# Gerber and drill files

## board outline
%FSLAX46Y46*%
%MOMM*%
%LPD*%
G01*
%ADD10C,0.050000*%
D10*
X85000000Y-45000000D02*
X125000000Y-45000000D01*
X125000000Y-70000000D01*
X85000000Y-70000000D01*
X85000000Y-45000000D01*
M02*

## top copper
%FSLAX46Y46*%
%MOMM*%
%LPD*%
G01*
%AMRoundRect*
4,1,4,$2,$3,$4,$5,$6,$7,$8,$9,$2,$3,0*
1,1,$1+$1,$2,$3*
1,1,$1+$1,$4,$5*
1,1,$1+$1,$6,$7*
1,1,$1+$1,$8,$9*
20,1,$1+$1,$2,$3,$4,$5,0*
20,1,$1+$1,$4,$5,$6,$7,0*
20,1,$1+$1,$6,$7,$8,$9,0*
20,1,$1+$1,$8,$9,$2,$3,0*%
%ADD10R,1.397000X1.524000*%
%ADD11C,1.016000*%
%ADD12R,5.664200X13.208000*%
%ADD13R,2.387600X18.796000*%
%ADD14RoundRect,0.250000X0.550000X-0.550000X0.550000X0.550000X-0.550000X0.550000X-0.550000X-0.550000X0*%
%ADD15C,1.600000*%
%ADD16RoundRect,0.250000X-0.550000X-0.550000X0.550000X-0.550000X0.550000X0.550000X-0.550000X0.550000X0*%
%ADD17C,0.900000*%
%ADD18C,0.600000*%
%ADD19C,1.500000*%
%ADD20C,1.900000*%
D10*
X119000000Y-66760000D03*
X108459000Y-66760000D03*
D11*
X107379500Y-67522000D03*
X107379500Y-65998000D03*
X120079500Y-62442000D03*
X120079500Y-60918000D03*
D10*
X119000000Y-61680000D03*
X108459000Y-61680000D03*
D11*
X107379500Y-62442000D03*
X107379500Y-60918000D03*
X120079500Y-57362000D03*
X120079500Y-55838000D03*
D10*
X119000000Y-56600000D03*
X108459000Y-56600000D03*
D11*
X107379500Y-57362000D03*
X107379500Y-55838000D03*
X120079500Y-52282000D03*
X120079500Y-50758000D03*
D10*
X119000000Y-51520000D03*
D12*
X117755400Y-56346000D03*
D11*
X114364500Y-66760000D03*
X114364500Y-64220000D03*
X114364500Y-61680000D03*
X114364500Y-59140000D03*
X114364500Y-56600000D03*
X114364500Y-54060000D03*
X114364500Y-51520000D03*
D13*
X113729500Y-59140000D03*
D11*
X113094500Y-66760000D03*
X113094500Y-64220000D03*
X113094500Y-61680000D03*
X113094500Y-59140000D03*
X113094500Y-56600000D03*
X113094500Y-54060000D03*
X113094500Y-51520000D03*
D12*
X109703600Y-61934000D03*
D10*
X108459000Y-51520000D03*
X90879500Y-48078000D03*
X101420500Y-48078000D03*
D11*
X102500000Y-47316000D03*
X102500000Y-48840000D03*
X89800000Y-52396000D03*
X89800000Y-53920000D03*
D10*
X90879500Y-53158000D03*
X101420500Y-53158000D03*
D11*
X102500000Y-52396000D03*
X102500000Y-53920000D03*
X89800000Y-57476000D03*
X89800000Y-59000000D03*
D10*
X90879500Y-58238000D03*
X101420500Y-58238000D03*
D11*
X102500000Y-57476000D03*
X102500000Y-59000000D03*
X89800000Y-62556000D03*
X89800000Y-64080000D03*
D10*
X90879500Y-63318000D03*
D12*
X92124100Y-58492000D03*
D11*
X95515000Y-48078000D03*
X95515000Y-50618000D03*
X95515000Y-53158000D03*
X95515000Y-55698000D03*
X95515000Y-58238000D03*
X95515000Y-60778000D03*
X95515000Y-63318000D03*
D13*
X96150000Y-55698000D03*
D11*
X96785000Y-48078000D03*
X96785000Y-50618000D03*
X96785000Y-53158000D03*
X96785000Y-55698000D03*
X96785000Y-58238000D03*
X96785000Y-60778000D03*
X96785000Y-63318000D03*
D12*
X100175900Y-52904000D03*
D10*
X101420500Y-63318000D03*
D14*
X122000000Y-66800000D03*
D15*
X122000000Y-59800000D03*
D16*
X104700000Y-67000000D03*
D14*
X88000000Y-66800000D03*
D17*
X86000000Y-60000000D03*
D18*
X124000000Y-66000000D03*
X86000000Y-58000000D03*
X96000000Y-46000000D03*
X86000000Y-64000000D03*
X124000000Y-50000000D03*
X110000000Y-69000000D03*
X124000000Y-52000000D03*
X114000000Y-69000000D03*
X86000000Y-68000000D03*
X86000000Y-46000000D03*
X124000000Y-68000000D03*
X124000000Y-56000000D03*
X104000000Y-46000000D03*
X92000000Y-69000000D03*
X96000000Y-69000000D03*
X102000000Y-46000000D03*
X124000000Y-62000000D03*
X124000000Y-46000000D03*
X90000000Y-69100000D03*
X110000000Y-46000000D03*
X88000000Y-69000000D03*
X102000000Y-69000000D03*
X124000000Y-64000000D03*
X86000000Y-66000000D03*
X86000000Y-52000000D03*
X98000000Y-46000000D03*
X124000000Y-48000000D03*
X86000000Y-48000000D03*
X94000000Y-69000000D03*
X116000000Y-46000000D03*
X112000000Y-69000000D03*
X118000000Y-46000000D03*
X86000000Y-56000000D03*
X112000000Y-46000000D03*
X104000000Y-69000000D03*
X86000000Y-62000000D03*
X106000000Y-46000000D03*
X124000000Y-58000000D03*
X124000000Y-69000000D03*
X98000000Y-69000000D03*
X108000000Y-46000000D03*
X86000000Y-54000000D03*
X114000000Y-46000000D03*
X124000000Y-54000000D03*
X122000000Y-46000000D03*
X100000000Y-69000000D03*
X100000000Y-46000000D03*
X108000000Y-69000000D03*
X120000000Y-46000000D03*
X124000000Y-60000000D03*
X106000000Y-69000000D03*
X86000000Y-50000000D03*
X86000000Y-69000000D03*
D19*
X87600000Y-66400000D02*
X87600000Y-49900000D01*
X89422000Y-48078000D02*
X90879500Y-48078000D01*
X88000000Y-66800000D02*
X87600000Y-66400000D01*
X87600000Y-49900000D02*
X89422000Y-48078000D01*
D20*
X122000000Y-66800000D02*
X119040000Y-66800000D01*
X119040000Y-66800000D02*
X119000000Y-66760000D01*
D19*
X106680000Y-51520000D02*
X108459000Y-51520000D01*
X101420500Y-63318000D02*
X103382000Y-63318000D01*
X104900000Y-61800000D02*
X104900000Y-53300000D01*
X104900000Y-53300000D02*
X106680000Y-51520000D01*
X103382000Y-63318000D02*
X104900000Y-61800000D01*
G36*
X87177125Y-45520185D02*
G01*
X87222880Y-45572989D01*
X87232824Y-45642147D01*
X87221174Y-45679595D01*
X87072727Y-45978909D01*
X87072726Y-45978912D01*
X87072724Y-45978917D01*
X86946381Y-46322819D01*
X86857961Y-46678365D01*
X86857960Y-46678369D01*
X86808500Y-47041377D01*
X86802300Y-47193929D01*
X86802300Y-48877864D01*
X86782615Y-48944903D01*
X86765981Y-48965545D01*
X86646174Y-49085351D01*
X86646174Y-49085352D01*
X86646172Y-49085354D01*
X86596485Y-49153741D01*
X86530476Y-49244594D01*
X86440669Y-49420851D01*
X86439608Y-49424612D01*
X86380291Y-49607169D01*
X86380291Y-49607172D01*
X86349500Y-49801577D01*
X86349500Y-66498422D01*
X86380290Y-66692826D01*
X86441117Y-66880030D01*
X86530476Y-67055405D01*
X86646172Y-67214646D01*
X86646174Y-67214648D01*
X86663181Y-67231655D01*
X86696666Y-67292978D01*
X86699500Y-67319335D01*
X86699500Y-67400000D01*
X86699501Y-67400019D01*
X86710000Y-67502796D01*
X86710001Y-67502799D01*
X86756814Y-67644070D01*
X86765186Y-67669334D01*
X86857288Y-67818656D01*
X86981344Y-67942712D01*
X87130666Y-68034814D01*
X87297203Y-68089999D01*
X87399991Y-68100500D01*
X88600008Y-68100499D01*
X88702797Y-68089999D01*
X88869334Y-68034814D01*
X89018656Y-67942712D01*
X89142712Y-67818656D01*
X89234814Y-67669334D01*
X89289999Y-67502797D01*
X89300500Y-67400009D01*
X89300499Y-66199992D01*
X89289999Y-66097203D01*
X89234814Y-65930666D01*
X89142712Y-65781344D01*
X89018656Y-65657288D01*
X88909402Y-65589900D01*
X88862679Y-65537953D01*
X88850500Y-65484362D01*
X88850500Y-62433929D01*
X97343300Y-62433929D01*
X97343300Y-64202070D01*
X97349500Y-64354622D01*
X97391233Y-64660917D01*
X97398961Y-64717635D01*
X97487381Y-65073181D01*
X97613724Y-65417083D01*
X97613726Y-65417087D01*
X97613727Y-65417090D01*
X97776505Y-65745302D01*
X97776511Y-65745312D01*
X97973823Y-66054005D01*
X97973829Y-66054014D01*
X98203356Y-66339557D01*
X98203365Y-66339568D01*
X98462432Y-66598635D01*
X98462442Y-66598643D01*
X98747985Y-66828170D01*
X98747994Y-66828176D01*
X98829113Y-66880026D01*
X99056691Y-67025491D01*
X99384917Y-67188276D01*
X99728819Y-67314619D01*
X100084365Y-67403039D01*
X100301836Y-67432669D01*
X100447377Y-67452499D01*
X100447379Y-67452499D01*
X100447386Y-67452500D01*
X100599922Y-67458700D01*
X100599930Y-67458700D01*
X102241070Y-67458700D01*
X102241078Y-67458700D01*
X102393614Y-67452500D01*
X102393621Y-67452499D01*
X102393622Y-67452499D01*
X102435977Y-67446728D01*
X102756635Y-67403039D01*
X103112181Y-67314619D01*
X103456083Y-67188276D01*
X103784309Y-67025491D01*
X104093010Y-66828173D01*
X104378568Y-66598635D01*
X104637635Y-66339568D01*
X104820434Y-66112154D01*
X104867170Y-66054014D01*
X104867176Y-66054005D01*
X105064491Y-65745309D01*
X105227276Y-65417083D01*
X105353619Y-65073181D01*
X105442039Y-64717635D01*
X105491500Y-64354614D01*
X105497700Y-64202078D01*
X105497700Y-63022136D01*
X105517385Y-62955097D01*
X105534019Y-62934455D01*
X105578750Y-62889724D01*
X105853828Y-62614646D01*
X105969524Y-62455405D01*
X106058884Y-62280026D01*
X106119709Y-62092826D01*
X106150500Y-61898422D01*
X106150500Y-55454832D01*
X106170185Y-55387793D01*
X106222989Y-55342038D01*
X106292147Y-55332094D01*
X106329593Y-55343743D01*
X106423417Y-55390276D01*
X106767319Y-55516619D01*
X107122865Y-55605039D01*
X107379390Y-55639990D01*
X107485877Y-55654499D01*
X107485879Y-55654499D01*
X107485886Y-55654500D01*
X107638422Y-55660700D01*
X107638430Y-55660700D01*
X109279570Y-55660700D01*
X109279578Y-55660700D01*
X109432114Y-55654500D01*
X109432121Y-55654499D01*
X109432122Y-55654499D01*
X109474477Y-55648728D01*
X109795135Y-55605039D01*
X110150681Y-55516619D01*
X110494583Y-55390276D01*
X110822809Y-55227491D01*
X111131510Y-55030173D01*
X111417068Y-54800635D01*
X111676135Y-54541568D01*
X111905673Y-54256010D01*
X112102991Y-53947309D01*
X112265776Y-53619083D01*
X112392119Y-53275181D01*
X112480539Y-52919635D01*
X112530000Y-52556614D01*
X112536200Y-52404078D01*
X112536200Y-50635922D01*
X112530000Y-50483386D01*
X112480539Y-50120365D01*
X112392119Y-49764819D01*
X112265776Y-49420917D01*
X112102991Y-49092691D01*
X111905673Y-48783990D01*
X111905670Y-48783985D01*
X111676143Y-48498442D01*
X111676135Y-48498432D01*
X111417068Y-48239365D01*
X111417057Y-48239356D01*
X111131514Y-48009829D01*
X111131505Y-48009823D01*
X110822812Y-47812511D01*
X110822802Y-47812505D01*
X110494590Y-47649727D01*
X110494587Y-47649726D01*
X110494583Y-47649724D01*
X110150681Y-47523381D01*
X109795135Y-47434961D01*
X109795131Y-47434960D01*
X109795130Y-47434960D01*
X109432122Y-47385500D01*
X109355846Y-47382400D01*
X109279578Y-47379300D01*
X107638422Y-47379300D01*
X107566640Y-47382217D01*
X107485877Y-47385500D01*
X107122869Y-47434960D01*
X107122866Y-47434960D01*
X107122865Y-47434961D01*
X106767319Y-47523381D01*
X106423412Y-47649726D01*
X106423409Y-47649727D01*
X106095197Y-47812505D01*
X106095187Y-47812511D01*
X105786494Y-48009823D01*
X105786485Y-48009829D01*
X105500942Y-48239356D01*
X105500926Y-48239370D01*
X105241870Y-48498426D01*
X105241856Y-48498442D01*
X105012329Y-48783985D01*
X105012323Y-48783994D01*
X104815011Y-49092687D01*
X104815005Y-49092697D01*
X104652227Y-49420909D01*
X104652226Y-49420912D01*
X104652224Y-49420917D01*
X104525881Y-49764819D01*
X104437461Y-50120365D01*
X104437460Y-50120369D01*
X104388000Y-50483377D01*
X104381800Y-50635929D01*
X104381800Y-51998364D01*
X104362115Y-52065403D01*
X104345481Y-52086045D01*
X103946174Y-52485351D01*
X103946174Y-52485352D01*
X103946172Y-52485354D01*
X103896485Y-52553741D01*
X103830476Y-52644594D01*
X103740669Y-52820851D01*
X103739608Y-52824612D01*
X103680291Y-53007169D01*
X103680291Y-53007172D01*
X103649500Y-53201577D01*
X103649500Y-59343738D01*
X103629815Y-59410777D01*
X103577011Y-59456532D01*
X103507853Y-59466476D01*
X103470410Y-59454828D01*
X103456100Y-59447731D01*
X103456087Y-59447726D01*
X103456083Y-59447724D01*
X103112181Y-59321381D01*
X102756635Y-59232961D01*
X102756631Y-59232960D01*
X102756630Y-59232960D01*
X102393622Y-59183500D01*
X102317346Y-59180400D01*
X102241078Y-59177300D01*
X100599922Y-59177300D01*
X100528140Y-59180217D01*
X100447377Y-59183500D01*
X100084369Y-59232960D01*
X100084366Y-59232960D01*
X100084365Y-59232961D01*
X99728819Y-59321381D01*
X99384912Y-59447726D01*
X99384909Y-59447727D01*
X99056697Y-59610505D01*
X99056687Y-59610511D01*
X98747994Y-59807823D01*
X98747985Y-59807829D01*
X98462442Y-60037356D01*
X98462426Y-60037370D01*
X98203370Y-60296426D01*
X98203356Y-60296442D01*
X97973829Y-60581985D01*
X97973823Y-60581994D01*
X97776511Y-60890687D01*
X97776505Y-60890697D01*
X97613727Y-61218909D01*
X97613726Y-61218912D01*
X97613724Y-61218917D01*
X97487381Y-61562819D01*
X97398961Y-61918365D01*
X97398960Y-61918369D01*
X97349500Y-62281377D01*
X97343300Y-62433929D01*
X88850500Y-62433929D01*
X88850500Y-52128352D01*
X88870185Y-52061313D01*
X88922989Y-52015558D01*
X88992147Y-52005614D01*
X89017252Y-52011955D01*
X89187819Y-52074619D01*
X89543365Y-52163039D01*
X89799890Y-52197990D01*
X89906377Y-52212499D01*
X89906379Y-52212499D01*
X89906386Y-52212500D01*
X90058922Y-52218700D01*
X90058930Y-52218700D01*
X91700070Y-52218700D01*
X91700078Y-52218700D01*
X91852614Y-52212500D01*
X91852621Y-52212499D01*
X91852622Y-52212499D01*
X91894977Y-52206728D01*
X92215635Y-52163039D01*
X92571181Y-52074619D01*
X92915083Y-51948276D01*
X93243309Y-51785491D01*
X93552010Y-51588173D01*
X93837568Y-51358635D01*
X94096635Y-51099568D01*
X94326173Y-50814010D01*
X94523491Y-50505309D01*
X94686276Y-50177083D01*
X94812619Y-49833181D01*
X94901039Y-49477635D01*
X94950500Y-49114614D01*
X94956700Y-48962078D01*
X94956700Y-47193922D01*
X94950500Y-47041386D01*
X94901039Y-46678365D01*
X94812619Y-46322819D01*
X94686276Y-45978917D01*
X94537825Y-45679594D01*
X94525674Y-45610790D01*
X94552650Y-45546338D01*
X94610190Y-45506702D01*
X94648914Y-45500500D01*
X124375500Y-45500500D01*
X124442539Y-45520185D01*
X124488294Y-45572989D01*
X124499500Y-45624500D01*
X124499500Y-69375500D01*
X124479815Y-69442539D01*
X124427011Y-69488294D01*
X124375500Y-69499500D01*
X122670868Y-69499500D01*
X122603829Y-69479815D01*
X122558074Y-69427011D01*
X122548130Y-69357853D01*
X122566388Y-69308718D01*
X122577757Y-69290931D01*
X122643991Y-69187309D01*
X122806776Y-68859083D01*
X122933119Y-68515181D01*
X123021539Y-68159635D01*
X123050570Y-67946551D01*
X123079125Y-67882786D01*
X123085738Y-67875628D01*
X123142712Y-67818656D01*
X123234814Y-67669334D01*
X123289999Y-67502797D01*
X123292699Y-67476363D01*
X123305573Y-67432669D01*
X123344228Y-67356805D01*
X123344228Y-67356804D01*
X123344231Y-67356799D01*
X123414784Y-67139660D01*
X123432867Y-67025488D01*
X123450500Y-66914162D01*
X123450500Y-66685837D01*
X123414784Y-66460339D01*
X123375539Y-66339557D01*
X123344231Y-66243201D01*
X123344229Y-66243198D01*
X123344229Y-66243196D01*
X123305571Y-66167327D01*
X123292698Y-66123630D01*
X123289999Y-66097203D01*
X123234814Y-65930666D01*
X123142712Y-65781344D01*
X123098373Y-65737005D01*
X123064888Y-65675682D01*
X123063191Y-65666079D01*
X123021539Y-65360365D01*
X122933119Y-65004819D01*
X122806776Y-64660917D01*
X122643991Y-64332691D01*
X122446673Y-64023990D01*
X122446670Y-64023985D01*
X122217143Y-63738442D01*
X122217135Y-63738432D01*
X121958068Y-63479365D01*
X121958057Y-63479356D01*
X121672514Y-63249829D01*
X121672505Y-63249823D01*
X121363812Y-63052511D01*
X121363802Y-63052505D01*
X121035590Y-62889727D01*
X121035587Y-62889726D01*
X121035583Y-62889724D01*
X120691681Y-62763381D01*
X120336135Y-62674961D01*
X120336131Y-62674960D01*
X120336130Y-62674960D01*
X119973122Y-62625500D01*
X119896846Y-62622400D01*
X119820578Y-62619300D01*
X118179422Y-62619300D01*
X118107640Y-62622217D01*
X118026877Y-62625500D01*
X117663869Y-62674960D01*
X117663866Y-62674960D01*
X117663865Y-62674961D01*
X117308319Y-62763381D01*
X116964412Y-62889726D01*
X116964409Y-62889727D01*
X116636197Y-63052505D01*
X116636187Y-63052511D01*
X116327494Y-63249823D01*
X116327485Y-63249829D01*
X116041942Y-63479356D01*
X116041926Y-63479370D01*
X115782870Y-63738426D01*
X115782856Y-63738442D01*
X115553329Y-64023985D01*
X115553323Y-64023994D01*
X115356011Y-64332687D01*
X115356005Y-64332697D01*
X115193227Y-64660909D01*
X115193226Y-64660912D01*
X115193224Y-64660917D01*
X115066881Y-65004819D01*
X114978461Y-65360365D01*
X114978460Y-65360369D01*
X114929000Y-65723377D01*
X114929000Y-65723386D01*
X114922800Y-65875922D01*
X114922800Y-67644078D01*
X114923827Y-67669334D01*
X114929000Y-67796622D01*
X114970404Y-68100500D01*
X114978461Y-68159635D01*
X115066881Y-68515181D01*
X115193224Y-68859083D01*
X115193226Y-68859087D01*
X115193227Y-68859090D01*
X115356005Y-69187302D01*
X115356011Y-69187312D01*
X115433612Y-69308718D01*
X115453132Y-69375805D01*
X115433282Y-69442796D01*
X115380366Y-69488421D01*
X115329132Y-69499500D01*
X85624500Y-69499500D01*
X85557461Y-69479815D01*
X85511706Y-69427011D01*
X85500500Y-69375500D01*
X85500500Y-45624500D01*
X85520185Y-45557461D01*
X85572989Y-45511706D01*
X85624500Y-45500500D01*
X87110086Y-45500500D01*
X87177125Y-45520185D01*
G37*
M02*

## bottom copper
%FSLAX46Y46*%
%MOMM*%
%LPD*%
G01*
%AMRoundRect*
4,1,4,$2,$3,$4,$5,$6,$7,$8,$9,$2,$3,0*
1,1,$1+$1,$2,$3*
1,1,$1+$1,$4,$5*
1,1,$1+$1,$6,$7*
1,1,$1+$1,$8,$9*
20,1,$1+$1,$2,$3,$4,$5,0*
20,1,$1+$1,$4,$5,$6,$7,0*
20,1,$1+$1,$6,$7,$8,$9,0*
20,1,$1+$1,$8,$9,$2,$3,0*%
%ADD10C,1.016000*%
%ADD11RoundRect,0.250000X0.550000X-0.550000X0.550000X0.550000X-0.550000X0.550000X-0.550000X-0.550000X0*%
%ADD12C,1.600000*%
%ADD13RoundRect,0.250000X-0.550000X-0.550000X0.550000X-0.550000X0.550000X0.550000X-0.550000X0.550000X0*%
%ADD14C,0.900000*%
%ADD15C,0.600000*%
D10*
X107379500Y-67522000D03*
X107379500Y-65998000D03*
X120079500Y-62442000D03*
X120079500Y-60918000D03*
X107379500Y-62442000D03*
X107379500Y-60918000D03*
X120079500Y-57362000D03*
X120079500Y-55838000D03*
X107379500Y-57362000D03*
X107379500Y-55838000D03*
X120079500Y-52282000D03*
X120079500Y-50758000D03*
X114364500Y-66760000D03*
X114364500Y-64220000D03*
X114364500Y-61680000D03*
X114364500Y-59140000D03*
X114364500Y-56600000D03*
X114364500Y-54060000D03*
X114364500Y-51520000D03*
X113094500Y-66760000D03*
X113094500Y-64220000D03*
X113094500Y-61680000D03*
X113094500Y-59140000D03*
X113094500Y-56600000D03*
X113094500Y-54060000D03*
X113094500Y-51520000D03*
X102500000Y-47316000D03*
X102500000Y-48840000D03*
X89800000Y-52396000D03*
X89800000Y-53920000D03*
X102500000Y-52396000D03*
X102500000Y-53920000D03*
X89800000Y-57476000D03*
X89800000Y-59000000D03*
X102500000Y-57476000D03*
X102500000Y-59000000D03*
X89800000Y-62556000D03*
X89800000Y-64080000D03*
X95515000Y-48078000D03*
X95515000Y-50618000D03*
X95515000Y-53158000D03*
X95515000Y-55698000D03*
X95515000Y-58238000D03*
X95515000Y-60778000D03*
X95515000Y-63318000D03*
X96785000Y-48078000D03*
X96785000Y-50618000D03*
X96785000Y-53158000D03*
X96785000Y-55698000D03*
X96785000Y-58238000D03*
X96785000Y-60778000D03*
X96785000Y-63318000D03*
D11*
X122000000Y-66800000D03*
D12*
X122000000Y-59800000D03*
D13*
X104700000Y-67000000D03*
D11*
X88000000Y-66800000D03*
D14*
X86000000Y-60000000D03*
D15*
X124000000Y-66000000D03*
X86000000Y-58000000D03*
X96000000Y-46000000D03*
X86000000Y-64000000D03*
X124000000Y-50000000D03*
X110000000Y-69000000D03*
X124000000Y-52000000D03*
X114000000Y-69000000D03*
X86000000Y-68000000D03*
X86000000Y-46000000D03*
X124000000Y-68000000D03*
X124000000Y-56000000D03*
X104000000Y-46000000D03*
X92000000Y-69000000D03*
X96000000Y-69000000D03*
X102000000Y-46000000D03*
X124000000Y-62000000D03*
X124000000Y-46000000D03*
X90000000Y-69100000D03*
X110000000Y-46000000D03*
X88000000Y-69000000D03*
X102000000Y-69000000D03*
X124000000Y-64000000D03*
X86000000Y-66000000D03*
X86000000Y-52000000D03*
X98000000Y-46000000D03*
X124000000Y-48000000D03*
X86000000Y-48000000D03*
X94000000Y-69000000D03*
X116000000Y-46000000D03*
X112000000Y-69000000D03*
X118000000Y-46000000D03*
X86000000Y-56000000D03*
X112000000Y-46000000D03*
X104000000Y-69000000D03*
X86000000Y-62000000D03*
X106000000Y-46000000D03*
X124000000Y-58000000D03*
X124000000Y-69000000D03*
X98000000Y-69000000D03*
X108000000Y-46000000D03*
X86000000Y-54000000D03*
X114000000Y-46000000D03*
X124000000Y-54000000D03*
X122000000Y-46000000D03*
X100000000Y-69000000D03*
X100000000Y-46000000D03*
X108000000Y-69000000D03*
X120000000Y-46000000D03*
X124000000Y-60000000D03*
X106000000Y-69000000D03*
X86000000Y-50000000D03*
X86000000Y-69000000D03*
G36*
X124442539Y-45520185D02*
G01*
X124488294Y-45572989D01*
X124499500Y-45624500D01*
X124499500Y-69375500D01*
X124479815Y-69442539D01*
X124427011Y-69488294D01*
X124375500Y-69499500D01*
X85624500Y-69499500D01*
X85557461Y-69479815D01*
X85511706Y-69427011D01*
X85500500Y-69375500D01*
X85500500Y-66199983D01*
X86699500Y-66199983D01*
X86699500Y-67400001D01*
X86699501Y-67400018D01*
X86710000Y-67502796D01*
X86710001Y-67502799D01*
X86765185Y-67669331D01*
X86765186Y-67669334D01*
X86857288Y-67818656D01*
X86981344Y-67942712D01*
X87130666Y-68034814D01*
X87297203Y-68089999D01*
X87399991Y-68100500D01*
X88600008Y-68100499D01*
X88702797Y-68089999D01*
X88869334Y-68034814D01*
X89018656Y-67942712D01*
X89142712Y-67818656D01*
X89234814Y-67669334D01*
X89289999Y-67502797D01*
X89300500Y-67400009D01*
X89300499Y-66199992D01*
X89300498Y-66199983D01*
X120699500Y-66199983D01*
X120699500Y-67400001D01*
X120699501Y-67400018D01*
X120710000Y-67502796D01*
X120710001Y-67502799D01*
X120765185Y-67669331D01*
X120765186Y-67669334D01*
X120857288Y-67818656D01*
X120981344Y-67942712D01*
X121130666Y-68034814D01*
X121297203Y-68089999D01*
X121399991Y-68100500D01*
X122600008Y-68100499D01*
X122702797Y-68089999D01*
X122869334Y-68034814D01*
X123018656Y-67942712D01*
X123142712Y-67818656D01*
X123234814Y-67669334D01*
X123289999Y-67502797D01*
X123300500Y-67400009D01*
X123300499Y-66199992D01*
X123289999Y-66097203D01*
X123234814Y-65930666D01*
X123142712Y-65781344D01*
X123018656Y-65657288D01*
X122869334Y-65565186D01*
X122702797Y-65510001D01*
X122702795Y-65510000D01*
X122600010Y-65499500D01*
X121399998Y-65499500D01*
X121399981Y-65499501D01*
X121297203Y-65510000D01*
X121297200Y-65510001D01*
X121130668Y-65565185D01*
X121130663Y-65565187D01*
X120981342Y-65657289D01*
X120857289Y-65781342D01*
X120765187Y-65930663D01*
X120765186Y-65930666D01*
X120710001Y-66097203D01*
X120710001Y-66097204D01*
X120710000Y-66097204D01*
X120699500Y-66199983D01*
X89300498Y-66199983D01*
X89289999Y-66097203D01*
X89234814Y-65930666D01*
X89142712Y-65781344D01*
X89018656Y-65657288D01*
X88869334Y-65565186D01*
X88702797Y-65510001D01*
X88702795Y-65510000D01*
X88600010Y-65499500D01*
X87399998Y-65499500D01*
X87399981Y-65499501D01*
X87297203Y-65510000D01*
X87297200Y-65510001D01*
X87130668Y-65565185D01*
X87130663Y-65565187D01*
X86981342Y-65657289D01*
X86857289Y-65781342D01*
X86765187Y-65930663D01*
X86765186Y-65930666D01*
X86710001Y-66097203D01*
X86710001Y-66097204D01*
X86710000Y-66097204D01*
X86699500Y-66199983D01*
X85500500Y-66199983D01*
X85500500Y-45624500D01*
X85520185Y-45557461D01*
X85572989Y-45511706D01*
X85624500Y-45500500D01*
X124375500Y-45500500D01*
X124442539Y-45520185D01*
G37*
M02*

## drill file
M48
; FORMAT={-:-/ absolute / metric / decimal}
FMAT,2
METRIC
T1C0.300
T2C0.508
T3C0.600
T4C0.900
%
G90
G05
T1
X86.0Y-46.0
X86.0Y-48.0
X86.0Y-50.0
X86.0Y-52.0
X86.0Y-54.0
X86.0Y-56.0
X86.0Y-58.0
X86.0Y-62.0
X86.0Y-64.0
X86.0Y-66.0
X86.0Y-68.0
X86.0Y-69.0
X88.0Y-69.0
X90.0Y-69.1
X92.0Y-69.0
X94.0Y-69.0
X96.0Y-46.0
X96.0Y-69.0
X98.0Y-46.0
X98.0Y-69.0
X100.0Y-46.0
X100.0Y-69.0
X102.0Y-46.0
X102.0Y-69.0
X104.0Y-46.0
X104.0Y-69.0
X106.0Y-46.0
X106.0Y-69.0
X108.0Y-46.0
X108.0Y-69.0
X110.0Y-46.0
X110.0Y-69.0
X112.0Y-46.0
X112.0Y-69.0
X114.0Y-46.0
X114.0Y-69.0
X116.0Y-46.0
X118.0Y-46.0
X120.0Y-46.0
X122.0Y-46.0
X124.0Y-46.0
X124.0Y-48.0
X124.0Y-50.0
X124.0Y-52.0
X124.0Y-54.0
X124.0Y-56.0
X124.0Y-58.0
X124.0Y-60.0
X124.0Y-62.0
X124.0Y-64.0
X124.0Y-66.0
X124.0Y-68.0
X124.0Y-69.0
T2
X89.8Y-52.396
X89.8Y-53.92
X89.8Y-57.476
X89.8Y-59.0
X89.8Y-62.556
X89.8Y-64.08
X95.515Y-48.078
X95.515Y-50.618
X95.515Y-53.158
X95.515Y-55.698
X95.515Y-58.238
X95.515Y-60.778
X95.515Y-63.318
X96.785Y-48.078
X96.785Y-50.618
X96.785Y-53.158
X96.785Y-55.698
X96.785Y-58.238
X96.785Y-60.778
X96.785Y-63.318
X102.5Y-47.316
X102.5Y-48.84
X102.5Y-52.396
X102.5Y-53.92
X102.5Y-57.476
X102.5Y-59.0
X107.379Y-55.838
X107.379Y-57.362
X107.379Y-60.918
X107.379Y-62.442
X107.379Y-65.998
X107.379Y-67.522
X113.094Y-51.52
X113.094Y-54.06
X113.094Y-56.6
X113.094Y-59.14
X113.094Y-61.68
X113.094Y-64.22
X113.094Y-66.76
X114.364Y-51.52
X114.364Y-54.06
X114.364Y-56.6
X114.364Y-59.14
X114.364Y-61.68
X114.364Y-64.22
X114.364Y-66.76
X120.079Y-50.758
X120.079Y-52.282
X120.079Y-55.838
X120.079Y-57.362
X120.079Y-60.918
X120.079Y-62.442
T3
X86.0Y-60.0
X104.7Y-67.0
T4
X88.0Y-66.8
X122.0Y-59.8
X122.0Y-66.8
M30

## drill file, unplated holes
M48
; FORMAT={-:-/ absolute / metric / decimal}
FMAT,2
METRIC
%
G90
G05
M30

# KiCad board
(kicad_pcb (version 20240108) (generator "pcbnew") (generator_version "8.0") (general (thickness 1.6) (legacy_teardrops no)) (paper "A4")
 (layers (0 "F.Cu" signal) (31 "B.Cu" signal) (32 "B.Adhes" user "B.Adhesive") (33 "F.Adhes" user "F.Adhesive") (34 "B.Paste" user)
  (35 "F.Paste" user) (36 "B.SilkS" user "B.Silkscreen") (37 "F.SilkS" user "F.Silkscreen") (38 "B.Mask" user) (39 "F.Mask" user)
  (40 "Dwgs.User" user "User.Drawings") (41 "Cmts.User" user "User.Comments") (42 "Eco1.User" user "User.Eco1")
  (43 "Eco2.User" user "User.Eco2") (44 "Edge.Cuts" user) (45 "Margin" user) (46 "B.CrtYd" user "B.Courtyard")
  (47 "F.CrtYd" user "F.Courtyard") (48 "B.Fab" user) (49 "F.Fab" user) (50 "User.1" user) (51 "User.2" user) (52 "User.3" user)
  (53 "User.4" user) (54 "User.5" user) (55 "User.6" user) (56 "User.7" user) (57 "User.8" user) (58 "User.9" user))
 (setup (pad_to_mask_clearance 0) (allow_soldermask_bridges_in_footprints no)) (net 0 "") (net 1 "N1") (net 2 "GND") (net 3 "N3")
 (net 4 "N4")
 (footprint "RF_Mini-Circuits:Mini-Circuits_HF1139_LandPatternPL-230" (layer "F.Cu") (at 113.7295 59.14 180)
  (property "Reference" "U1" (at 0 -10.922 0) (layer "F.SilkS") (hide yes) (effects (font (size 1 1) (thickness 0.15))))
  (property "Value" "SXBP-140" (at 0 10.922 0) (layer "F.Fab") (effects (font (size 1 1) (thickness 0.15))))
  (pad "1" smd rect (at -5.2705 -7.62 90) (size 1.524 1.397) (layers "F.Cu" "F.Paste" "F.Mask") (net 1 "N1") (clearance 3.3782))
  (pad "2" smd rect (at 5.2705 -7.62 90) (size 1.524 1.397) (layers "F.Cu" "F.Paste" "F.Mask") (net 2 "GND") (zone_connect 2))
  (pad "2" thru_hole circle (at 6.35 -8.382 90) (size 1.016 1.016) (drill 0.508) (layers "*.Cu") (remove_unused_layers no) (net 2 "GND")
   (zone_connect 2))
  (pad "2" thru_hole circle (at 6.35 -6.858 90) (size 1.016 1.016) (drill 0.508) (layers "*.Cu") (remove_unused_layers no) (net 2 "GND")
   (zone_connect 2))
  (pad "3" thru_hole circle (at -6.35 -3.302 90) (size 1.016 1.016) (drill 0.508) (layers "*.Cu") (remove_unused_layers no) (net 2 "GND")
   (zone_connect 2))
  (pad "3" thru_hole circle (at -6.35 -1.778 90) (size 1.016 1.016) (drill 0.508) (layers "*.Cu") (remove_unused_layers no) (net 2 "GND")
   (zone_connect 2))
  (pad "3" smd rect (at -5.2705 -2.54 90) (size 1.524 1.397) (layers "F.Cu" "F.Paste" "F.Mask") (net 2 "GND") (zone_connect 2))
  (pad "4" smd rect (at 5.2705 -2.54 90) (size 1.524 1.397) (layers "F.Cu" "F.Paste" "F.Mask") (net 2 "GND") (zone_connect 2))
  (pad "4" thru_hole circle (at 6.35 -3.302 90) (size 1.016 1.016) (drill 0.508) (layers "*.Cu") (remove_unused_layers no) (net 2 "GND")
   (zone_connect 2))
  (pad "4" thru_hole circle (at 6.35 -1.778 90) (size 1.016 1.016) (drill 0.508) (layers "*.Cu") (remove_unused_layers no) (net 2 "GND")
   (zone_connect 2))
  (pad "5" thru_hole circle (at -6.35 1.778 90) (size 1.016 1.016) (drill 0.508) (layers "*.Cu") (remove_unused_layers no) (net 2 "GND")
   (zone_connect 2))
  (pad "5" thru_hole circle (at -6.35 3.302 90) (size 1.016 1.016) (drill 0.508) (layers "*.Cu") (remove_unused_layers no) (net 2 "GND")
   (zone_connect 2))
  (pad "5" smd rect (at -5.2705 2.54 90) (size 1.524 1.397) (layers "F.Cu" "F.Paste" "F.Mask") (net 2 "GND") (zone_connect 2))
  (pad "6" smd rect (at 5.2705 2.54 90) (size 1.524 1.397) (layers "F.Cu" "F.Paste" "F.Mask") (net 2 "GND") (zone_connect 2))
  (pad "6" thru_hole circle (at 6.35 1.778 90) (size 1.016 1.016) (drill 0.508) (layers "*.Cu") (remove_unused_layers no) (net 2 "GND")
   (zone_connect 2))
  (pad "6" thru_hole circle (at 6.35 3.302 90) (size 1.016 1.016) (drill 0.508) (layers "*.Cu") (remove_unused_layers no) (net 2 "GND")
   (zone_connect 2))
  (pad "7" thru_hole circle (at -6.35 6.858 90) (size 1.016 1.016) (drill 0.508) (layers "*.Cu") (remove_unused_layers no) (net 2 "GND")
   (zone_connect 2))
  (pad "7" thru_hole circle (at -6.35 8.382 90) (size 1.016 1.016) (drill 0.508) (layers "*.Cu") (remove_unused_layers no) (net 2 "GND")
   (zone_connect 2))
  (pad "7" smd rect (at -5.2705 7.62 90) (size 1.524 1.397) (layers "F.Cu" "F.Paste" "F.Mask") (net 2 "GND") (zone_connect 2))
  (pad "7" smd rect (at -4.0259 2.794 90) (size 13.208 5.6642) (layers "F.Cu") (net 2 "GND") (zone_connect 2))
  (pad "7" thru_hole circle (at -0.635 -7.62 90) (size 1.016 1.016) (drill 0.508) (layers "*.Cu") (remove_unused_layers no) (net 2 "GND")
   (zone_connect 2))
  (pad "7" thru_hole circle (at -0.635 -5.08 90) (size 1.016 1.016) (drill 0.508) (layers "*.Cu") (remove_unused_layers no) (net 2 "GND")
   (zone_connect 2))
  (pad "7" thru_hole circle (at -0.635 -2.54 90) (size 1.016 1.016) (drill 0.508) (layers "*.Cu") (remove_unused_layers no) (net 2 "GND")
   (zone_connect 2))
  (pad "7" thru_hole circle (at -0.635 0 90) (size 1.016 1.016) (drill 0.508) (layers "*.Cu") (remove_unused_layers no) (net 2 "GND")
   (zone_connect 2))
  (pad "7" thru_hole circle (at -0.635 2.54 90) (size 1.016 1.016) (drill 0.508) (layers "*.Cu") (remove_unused_layers no) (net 2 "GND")
   (zone_connect 2))
  (pad "7" thru_hole circle (at -0.635 5.08 90) (size 1.016 1.016) (drill 0.508) (layers "*.Cu") (remove_unused_layers no) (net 2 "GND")
   (zone_connect 2))
  (pad "7" thru_hole circle (at -0.635 7.62 90) (size 1.016 1.016) (drill 0.508) (layers "*.Cu") (remove_unused_layers no) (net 2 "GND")
   (zone_connect 2))
  (pad "7" smd rect (at 0 0 90) (size 18.796 2.3876) (layers "F.Cu") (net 2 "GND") (zone_connect 2))
  (pad "7" thru_hole circle (at 0.635 -7.62 90) (size 1.016 1.016) (drill 0.508) (layers "*.Cu") (remove_unused_layers no) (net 2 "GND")
   (zone_connect 2))
  (pad "7" thru_hole circle (at 0.635 -5.08 90) (size 1.016 1.016) (drill 0.508) (layers "*.Cu") (remove_unused_layers no) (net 2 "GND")
   (zone_connect 2))
  (pad "7" thru_hole circle (at 0.635 -2.54 90) (size 1.016 1.016) (drill 0.508) (layers "*.Cu") (remove_unused_layers no) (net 2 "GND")
   (zone_connect 2))
  (pad "7" thru_hole circle (at 0.635 0 90) (size 1.016 1.016) (drill 0.508) (layers "*.Cu") (remove_unused_layers no) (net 2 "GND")
   (zone_connect 2))
  (pad "7" thru_hole circle (at 0.635 2.54 90) (size 1.016 1.016) (drill 0.508) (layers "*.Cu") (remove_unused_layers no) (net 2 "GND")
   (zone_connect 2))
  (pad "7" thru_hole circle (at 0.635 5.08 90) (size 1.016 1.016) (drill 0.508) (layers "*.Cu") (remove_unused_layers no) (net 2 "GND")
   (zone_connect 2))
  (pad "7" thru_hole circle (at 0.635 7.62 90) (size 1.016 1.016) (drill 0.508) (layers "*.Cu") (remove_unused_layers no) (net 2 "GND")
   (zone_connect 2))
  (pad "7" smd rect (at 4.0259 -2.794 90) (size 13.208 5.6642) (layers "F.Cu") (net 2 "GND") (zone_connect 2))
  (pad "8" smd rect (at 5.2705 7.62 90) (size 1.524 1.397) (layers "F.Cu" "F.Paste" "F.Mask") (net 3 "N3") (clearance 3.3782)))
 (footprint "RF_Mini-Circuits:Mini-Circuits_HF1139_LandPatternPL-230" (layer "F.Cu") (at 96.15 55.698)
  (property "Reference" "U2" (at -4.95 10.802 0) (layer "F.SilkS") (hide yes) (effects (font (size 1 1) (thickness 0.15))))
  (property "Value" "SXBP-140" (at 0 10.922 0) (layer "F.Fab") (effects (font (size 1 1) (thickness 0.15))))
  (pad "1" smd rect (at -5.2705 -7.62 270) (size 1.524 1.397) (layers "F.Cu" "F.Paste" "F.Mask") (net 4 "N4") (clearance 3.3782))
  (pad "2" smd rect (at 5.2705 -7.62 270) (size 1.524 1.397) (layers "F.Cu" "F.Paste" "F.Mask") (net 2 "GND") (zone_connect 2))
  (pad "2" thru_hole circle (at 6.35 -8.382 270) (size 1.016 1.016) (drill 0.508) (layers "*.Cu") (remove_unused_layers no) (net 2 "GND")
   (zone_connect 2))
  (pad "2" thru_hole circle (at 6.35 -6.858 270) (size 1.016 1.016) (drill 0.508) (layers "*.Cu") (remove_unused_layers no) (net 2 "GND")
   (zone_connect 2))
  (pad "3" thru_hole circle (at -6.35 -3.302 270) (size 1.016 1.016) (drill 0.508) (layers "*.Cu") (remove_unused_layers no) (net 2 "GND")
   (zone_connect 2))
  (pad "3" thru_hole circle (at -6.35 -1.778 270) (size 1.016 1.016) (drill 0.508) (layers "*.Cu") (remove_unused_layers no) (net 2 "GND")
   (zone_connect 2))
  (pad "3" smd rect (at -5.2705 -2.54 270) (size 1.524 1.397) (layers "F.Cu" "F.Paste" "F.Mask") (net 2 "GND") (zone_connect 2))
  (pad "4" smd rect (at 5.2705 -2.54 270) (size 1.524 1.397) (layers "F.Cu" "F.Paste" "F.Mask") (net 2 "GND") (zone_connect 2))
  (pad "4" thru_hole circle (at 6.35 -3.302 270) (size 1.016 1.016) (drill 0.508) (layers "*.Cu") (remove_unused_layers no) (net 2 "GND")
   (zone_connect 2))
  (pad "4" thru_hole circle (at 6.35 -1.778 270) (size 1.016 1.016) (drill 0.508) (layers "*.Cu") (remove_unused_layers no) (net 2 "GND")
   (zone_connect 2))
  (pad "5" thru_hole circle (at -6.35 1.778 270) (size 1.016 1.016) (drill 0.508) (layers "*.Cu") (remove_unused_layers no) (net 2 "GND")
   (zone_connect 2))
  (pad "5" thru_hole circle (at -6.35 3.302 270) (size 1.016 1.016) (drill 0.508) (layers "*.Cu") (remove_unused_layers no) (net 2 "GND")
   (zone_connect 2))
  (pad "5" smd rect (at -5.2705 2.54 270) (size 1.524 1.397) (layers "F.Cu" "F.Paste" "F.Mask") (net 2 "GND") (zone_connect 2))
  (pad "6" smd rect (at 5.2705 2.54 270) (size 1.524 1.397) (layers "F.Cu" "F.Paste" "F.Mask") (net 2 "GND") (zone_connect 2))
  (pad "6" thru_hole circle (at 6.35 1.778 270) (size 1.016 1.016) (drill 0.508) (layers "*.Cu") (remove_unused_layers no) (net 2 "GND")
   (zone_connect 2))
  (pad "6" thru_hole circle (at 6.35 3.302 270) (size 1.016 1.016) (drill 0.508) (layers "*.Cu") (remove_unused_layers no) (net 2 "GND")
   (zone_connect 2))
  (pad "7" thru_hole circle (at -6.35 6.858 270) (size 1.016 1.016) (drill 0.508) (layers "*.Cu") (remove_unused_layers no) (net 2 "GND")
   (zone_connect 2))
  (pad "7" thru_hole circle (at -6.35 8.382 270) (size 1.016 1.016) (drill 0.508) (layers "*.Cu") (remove_unused_layers no) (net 2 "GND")
   (zone_connect 2))
  (pad "7" smd rect (at -5.2705 7.62 270) (size 1.524 1.397) (layers "F.Cu" "F.Paste" "F.Mask") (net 2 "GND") (zone_connect 2))
  (pad "7" smd rect (at -4.0259 2.794 270) (size 13.208 5.6642) (layers "F.Cu") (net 2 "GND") (zone_connect 2))
  (pad "7" thru_hole circle (at -0.635 -7.62 270) (size 1.016 1.016) (drill 0.508) (layers "*.Cu") (remove_unused_layers no) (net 2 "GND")
   (zone_connect 2))
  (pad "7" thru_hole circle (at -0.635 -5.08 270) (size 1.016 1.016) (drill 0.508) (layers "*.Cu") (remove_unused_layers no) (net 2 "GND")
   (zone_connect 2))
  (pad "7" thru_hole circle (at -0.635 -2.54 270) (size 1.016 1.016) (drill 0.508) (layers "*.Cu") (remove_unused_layers no) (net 2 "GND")
   (zone_connect 2))
  (pad "7" thru_hole circle (at -0.635 0 270) (size 1.016 1.016) (drill 0.508) (layers "*.Cu") (remove_unused_layers no) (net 2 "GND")
   (zone_connect 2))
  (pad "7" thru_hole circle (at -0.635 2.54 270) (size 1.016 1.016) (drill 0.508) (layers "*.Cu") (remove_unused_layers no) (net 2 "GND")
   (zone_connect 2))
  (pad "7" thru_hole circle (at -0.635 5.08 270) (size 1.016 1.016) (drill 0.508) (layers "*.Cu") (remove_unused_layers no) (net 2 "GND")
   (zone_connect 2))
  (pad "7" thru_hole circle (at -0.635 7.62 270) (size 1.016 1.016) (drill 0.508) (layers "*.Cu") (remove_unused_layers no) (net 2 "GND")
   (zone_connect 2))
  (pad "7" smd rect (at 0 0 270) (size 18.796 2.3876) (layers "F.Cu") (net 2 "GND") (zone_connect 2))
  (pad "7" thru_hole circle (at 0.635 -7.62 270) (size 1.016 1.016) (drill 0.508) (layers "*.Cu") (remove_unused_layers no) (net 2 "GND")
   (zone_connect 2))
  (pad "7" thru_hole circle (at 0.635 -5.08 270) (size 1.016 1.016) (drill 0.508) (layers "*.Cu") (remove_unused_layers no) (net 2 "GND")
   (zone_connect 2))
  (pad "7" thru_hole circle (at 0.635 -2.54 270) (size 1.016 1.016) (drill 0.508) (layers "*.Cu") (remove_unused_layers no) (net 2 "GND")
   (zone_connect 2))
  (pad "7" thru_hole circle (at 0.635 0 270) (size 1.016 1.016) (drill 0.508) (layers "*.Cu") (remove_unused_layers no) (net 2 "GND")
   (zone_connect 2))
  (pad "7" thru_hole circle (at 0.635 2.54 270) (size 1.016 1.016) (drill 0.508) (layers "*.Cu") (remove_unused_layers no) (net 2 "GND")
   (zone_connect 2))
  (pad "7" thru_hole circle (at 0.635 5.08 270) (size 1.016 1.016) (drill 0.508) (layers "*.Cu") (remove_unused_layers no) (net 2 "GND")
   (zone_connect 2))
  (pad "7" thru_hole circle (at 0.635 7.62 270) (size 1.016 1.016) (drill 0.508) (layers "*.Cu") (remove_unused_layers no) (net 2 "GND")
   (zone_connect 2))
  (pad "7" smd rect (at 4.0259 -2.794 270) (size 13.208 5.6642) (layers "F.Cu") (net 2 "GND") (zone_connect 2))
  (pad "8" smd rect (at 5.2705 7.62 270) (size 1.524 1.397) (layers "F.Cu" "F.Paste" "F.Mask") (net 3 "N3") (clearance 3.3782)))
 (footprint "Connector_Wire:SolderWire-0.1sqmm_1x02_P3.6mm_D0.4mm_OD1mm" (layer "F.Cu") (at 122 66.8 90)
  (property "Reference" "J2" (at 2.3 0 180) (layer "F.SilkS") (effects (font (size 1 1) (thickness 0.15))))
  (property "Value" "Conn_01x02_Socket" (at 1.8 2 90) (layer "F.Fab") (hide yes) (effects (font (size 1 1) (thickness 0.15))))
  (pad "1" thru_hole roundrect (at 0 0 90) (size 1.6 1.6) (drill 0.9) (layers "*.Cu" "*.Mask") (remove_unused_layers no)
   (roundrect_rratio 0.15625) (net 1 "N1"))
  (pad "2" thru_hole circle (at 7 0 90) (size 1.6 1.6) (drill 0.9) (layers "*.Cu" "*.Mask") (remove_unused_layers no) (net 2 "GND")))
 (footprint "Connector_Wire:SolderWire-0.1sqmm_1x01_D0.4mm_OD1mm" (layer "F.Cu") (at 104.7 67)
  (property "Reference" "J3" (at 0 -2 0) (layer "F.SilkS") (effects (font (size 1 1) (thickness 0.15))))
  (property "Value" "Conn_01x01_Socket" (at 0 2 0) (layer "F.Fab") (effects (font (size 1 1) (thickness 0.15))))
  (pad "1" thru_hole roundrect (at 0 0) (size 1.6 1.6) (drill 0.6) (layers "*.Cu" "*.Mask") (remove_unused_layers no)
   (roundrect_rratio 0.15625) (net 2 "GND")))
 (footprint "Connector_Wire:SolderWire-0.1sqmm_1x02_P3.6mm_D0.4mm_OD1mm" (layer "F.Cu") (at 88 66.8 90)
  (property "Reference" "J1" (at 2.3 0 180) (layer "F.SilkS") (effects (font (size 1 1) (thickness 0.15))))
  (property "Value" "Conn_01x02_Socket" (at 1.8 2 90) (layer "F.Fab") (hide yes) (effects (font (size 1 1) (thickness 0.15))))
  (pad "1" thru_hole roundrect (at 0 0 90) (size 1.6 1.6) (drill 0.9) (layers "*.Cu" "*.Mask") (remove_unused_layers no)
   (roundrect_rratio 0.15625) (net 4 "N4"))
  (pad "2" thru_hole circle (at 6.8 -2 91.2) (size 0.9 0.9) (drill 0.6) (layers "*.Cu" "*.Mask") (remove_unused_layers no) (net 2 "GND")))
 (gr_rect (start 85 45) (end 125 70) (stroke (width 0.05) (type default)) (fill none) (layer "Edge.Cuts"))
 (segment (start 87.6 66.4) (end 87.6 49.9) (width 1.5) (layer "F.Cu") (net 4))
 (segment (start 89.422 48.078) (end 90.8795 48.078) (width 1.5) (layer "F.Cu") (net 4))
 (segment (start 88 66.8) (end 87.6 66.4) (width 1.5) (layer "F.Cu") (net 4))
 (segment (start 87.6 49.9) (end 89.422 48.078) (width 1.5) (layer "F.Cu") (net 4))
 (via (at 124 66) (size 0.6) (drill 0.3) (layers "F.Cu" "B.Cu") (free yes) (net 2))
 (via (at 86 58) (size 0.6) (drill 0.3) (layers "F.Cu" "B.Cu") (free yes) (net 2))
 (via (at 96 46) (size 0.6) (drill 0.3) (layers "F.Cu" "B.Cu") (free yes) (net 2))
 (via (at 86 64) (size 0.6) (drill 0.3) (layers "F.Cu" "B.Cu") (free yes) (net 2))
 (via (at 124 50) (size 0.6) (drill 0.3) (layers "F.Cu" "B.Cu") (free yes) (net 2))
 (via (at 110 69) (size 0.6) (drill 0.3) (layers "F.Cu" "B.Cu") (free yes) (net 2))
 (via (at 124 52) (size 0.6) (drill 0.3) (layers "F.Cu" "B.Cu") (free yes) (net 2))
 (via (at 114 69) (size 0.6) (drill 0.3) (layers "F.Cu" "B.Cu") (free yes) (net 2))
 (via (at 86 68) (size 0.6) (drill 0.3) (layers "F.Cu" "B.Cu") (free yes) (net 2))
 (via (at 86 46) (size 0.6) (drill 0.3) (layers "F.Cu" "B.Cu") (free yes) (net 2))
 (via (at 124 68) (size 0.6) (drill 0.3) (layers "F.Cu" "B.Cu") (free yes) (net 2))
 (via (at 124 56) (size 0.6) (drill 0.3) (layers "F.Cu" "B.Cu") (free yes) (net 2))
 (via (at 104 46) (size 0.6) (drill 0.3) (layers "F.Cu" "B.Cu") (free yes) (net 2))
 (via (at 92 69) (size 0.6) (drill 0.3) (layers "F.Cu" "B.Cu") (free yes) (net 2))
 (via (at 96 69) (size 0.6) (drill 0.3) (layers "F.Cu" "B.Cu") (free yes) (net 2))
 (via (at 102 46) (size 0.6) (drill 0.3) (layers "F.Cu" "B.Cu") (free yes) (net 2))
 (via (at 124 62) (size 0.6) (drill 0.3) (layers "F.Cu" "B.Cu") (free yes) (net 2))
 (via (at 124 46) (size 0.6) (drill 0.3) (layers "F.Cu" "B.Cu") (free yes) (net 2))
 (via (at 90 69.1) (size 0.6) (drill 0.3) (layers "F.Cu" "B.Cu") (free yes) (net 2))
 (via (at 110 46) (size 0.6) (drill 0.3) (layers "F.Cu" "B.Cu") (free yes) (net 2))
 (via (at 88 69) (size 0.6) (drill 0.3) (layers "F.Cu" "B.Cu") (free yes) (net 2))
 (via (at 102 69) (size 0.6) (drill 0.3) (layers "F.Cu" "B.Cu") (free yes) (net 2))
 (via (at 124 64) (size 0.6) (drill 0.3) (layers "F.Cu" "B.Cu") (free yes) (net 2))
 (via (at 86 66) (size 0.6) (drill 0.3) (layers "F.Cu" "B.Cu") (free yes) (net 2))
 (via (at 86 52) (size 0.6) (drill 0.3) (layers "F.Cu" "B.Cu") (free yes) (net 2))
 (via (at 98 46) (size 0.6) (drill 0.3) (layers "F.Cu" "B.Cu") (free yes) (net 2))
 (via (at 124 48) (size 0.6) (drill 0.3) (layers "F.Cu" "B.Cu") (free yes) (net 2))
 (via (at 86 48) (size 0.6) (drill 0.3) (layers "F.Cu" "B.Cu") (free yes) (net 2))
 (via (at 94 69) (size 0.6) (drill 0.3) (layers "F.Cu" "B.Cu") (free yes) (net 2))
 (via (at 116 46) (size 0.6) (drill 0.3) (layers "F.Cu" "B.Cu") (free yes) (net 2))
 (via (at 112 69) (size 0.6) (drill 0.3) (layers "F.Cu" "B.Cu") (free yes) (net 2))
 (via (at 118 46) (size 0.6) (drill 0.3) (layers "F.Cu" "B.Cu") (free yes) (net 2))
 (via (at 86 56) (size 0.6) (drill 0.3) (layers "F.Cu" "B.Cu") (free yes) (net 2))
 (via (at 112 46) (size 0.6) (drill 0.3) (layers "F.Cu" "B.Cu") (free yes) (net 2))
 (via (at 104 69) (size 0.6) (drill 0.3) (layers "F.Cu" "B.Cu") (free yes) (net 2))
 (via (at 86 62) (size 0.6) (drill 0.3) (layers "F.Cu" "B.Cu") (free yes) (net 2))
 (via (at 106 46) (size 0.6) (drill 0.3) (layers "F.Cu" "B.Cu") (free yes) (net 2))
 (via (at 124 58) (size 0.6) (drill 0.3) (layers "F.Cu" "B.Cu") (free yes) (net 2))
 (via (at 124 69) (size 0.6) (drill 0.3) (layers "F.Cu" "B.Cu") (free yes) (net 2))
 (via (at 98 69) (size 0.6) (drill 0.3) (layers "F.Cu" "B.Cu") (free yes) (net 2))
 (via (at 108 46) (size 0.6) (drill 0.3) (layers "F.Cu" "B.Cu") (free yes) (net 2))
 (via (at 86 54) (size 0.6) (drill 0.3) (layers "F.Cu" "B.Cu") (free yes) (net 2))
 (via (at 114 46) (size 0.6) (drill 0.3) (layers "F.Cu" "B.Cu") (free yes) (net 2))
 (via (at 124 54) (size 0.6) (drill 0.3) (layers "F.Cu" "B.Cu") (free yes) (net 2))
 (via (at 122 46) (size 0.6) (drill 0.3) (layers "F.Cu" "B.Cu") (free yes) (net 2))
 (via (at 100 69) (size 0.6) (drill 0.3) (layers "F.Cu" "B.Cu") (free yes) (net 2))
 (via (at 100 46) (size 0.6) (drill 0.3) (layers "F.Cu" "B.Cu") (free yes) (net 2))
 (via (at 108 69) (size 0.6) (drill 0.3) (layers "F.Cu" "B.Cu") (free yes) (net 2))
 (via (at 120 46) (size 0.6) (drill 0.3) (layers "F.Cu" "B.Cu") (free yes) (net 2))
 (via (at 124 60) (size 0.6) (drill 0.3) (layers "F.Cu" "B.Cu") (free yes) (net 2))
 (via (at 106 69) (size 0.6) (drill 0.3) (layers "F.Cu" "B.Cu") (free yes) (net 2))
 (via (at 86 50) (size 0.6) (drill 0.3) (layers "F.Cu" "B.Cu") (free yes) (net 2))
 (via (at 86 69) (size 0.6) (drill 0.3) (layers "F.Cu" "B.Cu") (free yes) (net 2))
 (segment (start 122 66.8) (end 119.04 66.8) (width 1.9) (layer "F.Cu") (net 1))
 (segment (start 119.04 66.8) (end 119 66.76) (width 1.9) (layer "F.Cu") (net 1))
 (segment (start 106.68 51.52) (end 108.459 51.52) (width 1.5) (layer "F.Cu") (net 3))
 (segment (start 101.4205 63.318) (end 103.382 63.318) (width 1.5) (layer "F.Cu") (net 3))
 (segment (start 104.9 61.8) (end 104.9 53.3) (width 1.5) (layer "F.Cu") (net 3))
 (segment (start 104.9 53.3) (end 106.68 51.52) (width 1.5) (layer "F.Cu") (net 3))
 (segment (start 103.382 63.318) (end 104.9 61.8) (width 1.5) (layer "F.Cu") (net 3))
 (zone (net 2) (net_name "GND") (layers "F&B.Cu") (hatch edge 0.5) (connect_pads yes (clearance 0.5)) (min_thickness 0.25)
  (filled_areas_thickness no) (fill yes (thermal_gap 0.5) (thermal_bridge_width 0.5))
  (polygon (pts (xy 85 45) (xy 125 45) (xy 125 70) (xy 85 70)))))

